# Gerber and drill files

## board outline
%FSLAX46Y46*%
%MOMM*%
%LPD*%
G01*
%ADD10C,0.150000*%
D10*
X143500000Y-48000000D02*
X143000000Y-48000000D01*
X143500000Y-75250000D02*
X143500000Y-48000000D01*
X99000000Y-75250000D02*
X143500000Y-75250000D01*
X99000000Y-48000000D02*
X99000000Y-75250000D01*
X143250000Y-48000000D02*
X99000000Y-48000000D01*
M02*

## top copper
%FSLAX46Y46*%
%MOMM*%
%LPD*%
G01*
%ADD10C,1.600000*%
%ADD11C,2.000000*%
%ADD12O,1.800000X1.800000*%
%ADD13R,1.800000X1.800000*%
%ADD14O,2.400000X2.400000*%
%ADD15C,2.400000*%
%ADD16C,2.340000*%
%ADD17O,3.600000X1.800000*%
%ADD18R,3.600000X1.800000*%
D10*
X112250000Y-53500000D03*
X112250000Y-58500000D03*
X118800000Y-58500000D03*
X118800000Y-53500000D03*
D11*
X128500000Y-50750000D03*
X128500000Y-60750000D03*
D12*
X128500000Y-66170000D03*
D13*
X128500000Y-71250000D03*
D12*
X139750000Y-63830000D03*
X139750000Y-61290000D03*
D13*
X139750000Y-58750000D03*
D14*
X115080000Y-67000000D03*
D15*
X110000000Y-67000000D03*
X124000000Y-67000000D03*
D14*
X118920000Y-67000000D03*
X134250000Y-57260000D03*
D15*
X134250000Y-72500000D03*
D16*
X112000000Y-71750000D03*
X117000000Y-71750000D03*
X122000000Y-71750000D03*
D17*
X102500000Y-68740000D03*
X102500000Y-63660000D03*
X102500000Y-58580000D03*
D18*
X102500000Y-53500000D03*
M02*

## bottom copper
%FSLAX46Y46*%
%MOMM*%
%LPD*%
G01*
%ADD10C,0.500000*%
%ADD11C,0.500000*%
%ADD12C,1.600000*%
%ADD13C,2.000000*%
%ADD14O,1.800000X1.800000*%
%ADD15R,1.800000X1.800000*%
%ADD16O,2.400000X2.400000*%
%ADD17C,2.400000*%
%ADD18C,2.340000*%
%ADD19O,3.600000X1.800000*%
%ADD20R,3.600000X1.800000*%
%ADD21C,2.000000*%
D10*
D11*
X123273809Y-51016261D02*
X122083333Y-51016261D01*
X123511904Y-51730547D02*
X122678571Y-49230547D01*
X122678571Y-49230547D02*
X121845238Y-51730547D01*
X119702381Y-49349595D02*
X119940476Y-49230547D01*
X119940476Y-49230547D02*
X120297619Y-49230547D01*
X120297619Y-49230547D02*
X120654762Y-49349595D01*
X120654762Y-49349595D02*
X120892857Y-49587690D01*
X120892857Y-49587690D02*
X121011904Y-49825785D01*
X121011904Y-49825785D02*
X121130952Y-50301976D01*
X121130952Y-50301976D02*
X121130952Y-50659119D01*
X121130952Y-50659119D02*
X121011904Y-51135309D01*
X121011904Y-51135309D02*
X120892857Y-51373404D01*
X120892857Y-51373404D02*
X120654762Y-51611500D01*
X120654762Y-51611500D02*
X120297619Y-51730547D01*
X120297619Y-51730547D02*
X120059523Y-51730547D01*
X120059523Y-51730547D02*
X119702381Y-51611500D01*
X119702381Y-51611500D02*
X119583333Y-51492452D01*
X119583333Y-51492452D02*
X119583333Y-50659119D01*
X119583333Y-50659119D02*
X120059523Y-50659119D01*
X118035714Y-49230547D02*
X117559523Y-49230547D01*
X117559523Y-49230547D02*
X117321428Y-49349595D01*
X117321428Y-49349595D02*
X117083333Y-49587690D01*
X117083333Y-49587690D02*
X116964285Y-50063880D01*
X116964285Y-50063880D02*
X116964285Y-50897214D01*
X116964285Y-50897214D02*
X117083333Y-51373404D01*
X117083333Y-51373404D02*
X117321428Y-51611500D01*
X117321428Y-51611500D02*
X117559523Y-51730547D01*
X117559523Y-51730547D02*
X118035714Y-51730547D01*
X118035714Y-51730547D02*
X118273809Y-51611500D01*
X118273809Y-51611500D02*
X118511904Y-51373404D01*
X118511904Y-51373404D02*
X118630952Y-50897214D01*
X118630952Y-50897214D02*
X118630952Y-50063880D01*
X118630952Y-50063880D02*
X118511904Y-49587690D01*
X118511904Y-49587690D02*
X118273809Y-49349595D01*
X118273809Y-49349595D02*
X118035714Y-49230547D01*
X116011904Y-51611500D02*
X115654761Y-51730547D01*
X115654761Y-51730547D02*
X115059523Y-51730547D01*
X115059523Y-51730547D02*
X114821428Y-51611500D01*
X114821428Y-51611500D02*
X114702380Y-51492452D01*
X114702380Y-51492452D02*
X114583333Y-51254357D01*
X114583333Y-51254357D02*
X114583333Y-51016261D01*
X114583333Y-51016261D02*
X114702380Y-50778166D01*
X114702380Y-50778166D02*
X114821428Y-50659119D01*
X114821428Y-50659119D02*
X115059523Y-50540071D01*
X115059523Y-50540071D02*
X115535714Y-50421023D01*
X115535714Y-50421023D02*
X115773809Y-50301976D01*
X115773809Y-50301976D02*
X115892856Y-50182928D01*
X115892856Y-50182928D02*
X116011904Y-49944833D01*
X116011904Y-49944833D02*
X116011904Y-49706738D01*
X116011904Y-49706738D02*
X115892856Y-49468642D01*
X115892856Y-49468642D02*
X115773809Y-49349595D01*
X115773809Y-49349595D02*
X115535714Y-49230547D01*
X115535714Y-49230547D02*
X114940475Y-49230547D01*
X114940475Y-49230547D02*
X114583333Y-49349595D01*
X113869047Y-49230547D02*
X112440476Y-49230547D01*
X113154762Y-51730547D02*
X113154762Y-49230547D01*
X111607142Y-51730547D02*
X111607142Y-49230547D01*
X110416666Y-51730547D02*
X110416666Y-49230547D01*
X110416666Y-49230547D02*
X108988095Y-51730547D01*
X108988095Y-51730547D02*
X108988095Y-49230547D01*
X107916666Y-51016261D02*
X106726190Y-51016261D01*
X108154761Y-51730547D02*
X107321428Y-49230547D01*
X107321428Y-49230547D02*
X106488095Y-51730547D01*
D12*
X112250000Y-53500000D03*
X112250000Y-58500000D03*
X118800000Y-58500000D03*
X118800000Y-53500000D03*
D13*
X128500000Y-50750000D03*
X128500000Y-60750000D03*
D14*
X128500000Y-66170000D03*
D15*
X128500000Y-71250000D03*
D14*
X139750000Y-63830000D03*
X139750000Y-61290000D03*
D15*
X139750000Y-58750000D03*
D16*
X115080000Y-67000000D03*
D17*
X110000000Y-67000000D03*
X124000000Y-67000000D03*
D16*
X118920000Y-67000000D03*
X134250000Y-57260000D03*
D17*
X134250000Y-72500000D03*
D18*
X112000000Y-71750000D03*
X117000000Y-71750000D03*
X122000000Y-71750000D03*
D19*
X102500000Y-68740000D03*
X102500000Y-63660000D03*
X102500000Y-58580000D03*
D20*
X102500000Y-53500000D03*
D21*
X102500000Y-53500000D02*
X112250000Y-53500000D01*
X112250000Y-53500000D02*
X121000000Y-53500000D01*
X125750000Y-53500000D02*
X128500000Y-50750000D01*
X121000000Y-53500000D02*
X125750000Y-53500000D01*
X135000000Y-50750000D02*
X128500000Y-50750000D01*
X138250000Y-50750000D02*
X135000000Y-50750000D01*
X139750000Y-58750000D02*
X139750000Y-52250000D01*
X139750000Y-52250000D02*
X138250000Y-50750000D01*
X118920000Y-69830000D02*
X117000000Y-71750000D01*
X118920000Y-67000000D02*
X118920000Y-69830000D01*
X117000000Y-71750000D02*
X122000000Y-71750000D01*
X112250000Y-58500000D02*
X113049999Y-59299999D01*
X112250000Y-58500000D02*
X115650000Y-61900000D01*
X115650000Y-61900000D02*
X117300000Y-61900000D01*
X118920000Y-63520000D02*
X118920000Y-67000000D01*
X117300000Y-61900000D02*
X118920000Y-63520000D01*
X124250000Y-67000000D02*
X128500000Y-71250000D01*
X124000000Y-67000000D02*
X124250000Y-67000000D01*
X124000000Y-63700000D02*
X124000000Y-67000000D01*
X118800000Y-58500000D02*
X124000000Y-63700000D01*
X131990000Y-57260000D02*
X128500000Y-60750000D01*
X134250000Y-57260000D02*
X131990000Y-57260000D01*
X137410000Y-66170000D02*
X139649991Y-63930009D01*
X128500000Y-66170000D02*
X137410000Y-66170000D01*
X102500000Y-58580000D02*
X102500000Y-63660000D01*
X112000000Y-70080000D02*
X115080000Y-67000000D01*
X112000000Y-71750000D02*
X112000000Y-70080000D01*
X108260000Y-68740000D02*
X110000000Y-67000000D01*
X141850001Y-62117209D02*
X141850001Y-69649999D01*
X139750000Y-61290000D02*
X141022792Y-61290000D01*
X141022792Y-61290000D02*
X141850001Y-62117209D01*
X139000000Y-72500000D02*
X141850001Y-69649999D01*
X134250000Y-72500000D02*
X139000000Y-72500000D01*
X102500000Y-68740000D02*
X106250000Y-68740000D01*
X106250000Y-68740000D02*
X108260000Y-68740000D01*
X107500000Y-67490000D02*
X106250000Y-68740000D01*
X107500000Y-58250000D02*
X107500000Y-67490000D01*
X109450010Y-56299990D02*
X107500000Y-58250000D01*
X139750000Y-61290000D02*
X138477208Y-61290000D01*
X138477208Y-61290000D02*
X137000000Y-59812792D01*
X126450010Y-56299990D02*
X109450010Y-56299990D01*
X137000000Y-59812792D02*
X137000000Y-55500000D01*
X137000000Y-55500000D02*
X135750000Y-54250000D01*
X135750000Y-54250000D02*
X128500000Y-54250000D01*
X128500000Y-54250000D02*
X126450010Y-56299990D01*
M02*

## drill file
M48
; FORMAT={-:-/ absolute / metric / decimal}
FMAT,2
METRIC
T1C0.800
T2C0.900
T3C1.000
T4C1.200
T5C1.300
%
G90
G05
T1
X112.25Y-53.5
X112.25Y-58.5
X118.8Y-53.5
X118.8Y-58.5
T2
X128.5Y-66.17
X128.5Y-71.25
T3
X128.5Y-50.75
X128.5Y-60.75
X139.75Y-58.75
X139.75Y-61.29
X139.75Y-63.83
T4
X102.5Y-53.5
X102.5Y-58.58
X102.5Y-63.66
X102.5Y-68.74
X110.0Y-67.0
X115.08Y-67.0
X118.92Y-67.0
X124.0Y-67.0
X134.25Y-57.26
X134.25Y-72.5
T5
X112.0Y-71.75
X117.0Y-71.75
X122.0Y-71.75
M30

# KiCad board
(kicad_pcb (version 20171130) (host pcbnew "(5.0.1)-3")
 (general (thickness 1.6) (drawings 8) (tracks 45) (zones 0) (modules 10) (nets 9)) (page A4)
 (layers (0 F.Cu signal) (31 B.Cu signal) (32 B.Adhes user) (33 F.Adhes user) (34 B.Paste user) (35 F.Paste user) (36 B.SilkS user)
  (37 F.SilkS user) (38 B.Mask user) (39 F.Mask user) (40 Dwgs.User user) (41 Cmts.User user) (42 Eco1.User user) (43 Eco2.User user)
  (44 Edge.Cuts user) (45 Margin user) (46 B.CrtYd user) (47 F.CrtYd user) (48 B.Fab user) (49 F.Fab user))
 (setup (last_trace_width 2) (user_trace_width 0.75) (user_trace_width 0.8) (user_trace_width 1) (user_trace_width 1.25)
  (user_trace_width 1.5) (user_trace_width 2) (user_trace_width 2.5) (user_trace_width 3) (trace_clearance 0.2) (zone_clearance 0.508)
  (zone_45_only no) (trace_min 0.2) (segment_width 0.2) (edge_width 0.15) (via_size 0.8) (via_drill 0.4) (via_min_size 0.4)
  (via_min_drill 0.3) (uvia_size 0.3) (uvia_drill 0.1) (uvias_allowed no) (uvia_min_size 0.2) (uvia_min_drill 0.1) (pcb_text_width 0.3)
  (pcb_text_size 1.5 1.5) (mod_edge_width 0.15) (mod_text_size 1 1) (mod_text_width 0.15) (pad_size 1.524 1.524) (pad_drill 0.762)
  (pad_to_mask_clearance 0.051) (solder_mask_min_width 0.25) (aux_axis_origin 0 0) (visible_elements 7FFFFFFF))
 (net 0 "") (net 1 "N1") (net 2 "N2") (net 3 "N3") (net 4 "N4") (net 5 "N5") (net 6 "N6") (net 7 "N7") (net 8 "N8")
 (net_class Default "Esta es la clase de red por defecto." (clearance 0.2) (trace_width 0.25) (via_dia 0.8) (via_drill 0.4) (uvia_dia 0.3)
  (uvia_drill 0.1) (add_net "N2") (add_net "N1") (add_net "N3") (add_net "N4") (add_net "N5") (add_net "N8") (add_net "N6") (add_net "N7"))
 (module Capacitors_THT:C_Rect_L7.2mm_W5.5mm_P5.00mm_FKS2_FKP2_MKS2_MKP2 (layer F.Cu) (at 112.25 58.5 90)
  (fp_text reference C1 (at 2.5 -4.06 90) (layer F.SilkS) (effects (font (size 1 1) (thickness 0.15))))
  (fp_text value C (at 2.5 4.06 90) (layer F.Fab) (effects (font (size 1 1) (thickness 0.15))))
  (pad 2 thru_hole circle (at 5 0 90) (size 1.6 1.6) (drill 0.8) (layers *.Cu *.Mask) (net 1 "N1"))
  (pad 1 thru_hole circle (at 0 0 90) (size 1.6 1.6) (drill 0.8) (layers *.Cu *.Mask) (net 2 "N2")))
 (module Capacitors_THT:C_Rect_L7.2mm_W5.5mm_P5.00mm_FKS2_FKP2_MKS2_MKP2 (layer F.Cu) (at 118.8 58.5 90)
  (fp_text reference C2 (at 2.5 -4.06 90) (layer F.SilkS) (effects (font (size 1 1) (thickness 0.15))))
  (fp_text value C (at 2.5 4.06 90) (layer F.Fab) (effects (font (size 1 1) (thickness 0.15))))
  (pad 1 thru_hole circle (at 0 0 90) (size 1.6 1.6) (drill 0.8) (layers *.Cu *.Mask) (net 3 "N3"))
  (pad 2 thru_hole circle (at 5 0 90) (size 1.6 1.6) (drill 0.8) (layers *.Cu *.Mask) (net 1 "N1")))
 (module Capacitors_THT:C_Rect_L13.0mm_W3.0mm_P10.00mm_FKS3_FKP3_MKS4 (layer F.Cu) (at 128.5 60.75 90)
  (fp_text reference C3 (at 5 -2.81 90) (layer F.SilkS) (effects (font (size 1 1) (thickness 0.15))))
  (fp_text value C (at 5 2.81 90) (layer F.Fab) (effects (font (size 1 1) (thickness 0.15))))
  (pad 2 thru_hole circle (at 10 0 90) (size 2 2) (drill 1) (layers *.Cu *.Mask) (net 1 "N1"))
  (pad 1 thru_hole circle (at 0 0 90) (size 2 2) (drill 1) (layers *.Cu *.Mask) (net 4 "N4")))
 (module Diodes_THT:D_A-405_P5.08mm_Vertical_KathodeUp (layer F.Cu) (at 128.5 71.25 90)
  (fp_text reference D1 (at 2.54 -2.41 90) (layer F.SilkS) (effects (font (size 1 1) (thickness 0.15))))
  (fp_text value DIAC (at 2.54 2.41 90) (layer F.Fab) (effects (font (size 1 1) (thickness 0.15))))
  (pad 2 thru_hole oval (at 5.08 0 90) (size 1.8 1.8) (drill 0.9) (layers *.Cu *.Mask) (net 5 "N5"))
  (pad 1 thru_hole rect (at 0 0 90) (size 1.8 1.8) (drill 0.9) (layers *.Cu *.Mask) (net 3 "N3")))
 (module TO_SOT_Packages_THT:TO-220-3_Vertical (layer F.Cu) (at 139.75 58.75 270)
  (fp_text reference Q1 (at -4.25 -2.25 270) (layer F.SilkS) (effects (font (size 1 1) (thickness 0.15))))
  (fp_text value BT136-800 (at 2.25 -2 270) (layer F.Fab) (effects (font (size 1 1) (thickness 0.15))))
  (pad 3 thru_hole oval (at 5.08 0 270) (size 1.8 1.8) (drill 1) (layers *.Cu *.Mask) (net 5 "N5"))
  (pad 2 thru_hole oval (at 2.54 0 270) (size 1.8 1.8) (drill 1) (layers *.Cu *.Mask) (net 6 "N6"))
  (pad 1 thru_hole rect (at 0 0 270) (size 1.8 1.8) (drill 1) (layers *.Cu *.Mask) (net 1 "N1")))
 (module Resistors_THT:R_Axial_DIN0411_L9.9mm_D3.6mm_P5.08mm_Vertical (layer F.Cu) (at 110 67)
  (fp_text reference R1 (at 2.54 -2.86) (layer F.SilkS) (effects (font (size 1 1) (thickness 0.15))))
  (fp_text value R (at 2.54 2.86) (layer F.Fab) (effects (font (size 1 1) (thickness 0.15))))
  (pad 2 thru_hole oval (at 5.08 0) (size 2.4 2.4) (drill 1.2) (layers *.Cu *.Mask) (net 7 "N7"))
  (pad 1 thru_hole circle (at 0 0) (size 2.4 2.4) (drill 1.2) (layers *.Cu *.Mask) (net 6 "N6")))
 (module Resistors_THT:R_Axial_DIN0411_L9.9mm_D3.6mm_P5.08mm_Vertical (layer F.Cu) (at 124 67 180)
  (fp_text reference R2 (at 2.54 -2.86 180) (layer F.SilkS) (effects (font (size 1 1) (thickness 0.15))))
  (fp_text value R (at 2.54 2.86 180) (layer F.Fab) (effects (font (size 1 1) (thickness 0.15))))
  (pad 1 thru_hole circle (at 0 0 180) (size 2.4 2.4) (drill 1.2) (layers *.Cu *.Mask) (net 3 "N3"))
  (pad 2 thru_hole oval (at 5.08 0 180) (size 2.4 2.4) (drill 1.2) (layers *.Cu *.Mask) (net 2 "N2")))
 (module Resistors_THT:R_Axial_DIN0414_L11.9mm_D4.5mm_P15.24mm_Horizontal (layer F.Cu) (at 134.25 72.5 90)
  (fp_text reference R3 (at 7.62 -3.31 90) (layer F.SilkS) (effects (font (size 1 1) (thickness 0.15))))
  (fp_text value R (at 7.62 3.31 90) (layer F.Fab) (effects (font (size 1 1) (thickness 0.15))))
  (pad 2 thru_hole oval (at 15.24 0 90) (size 2.4 2.4) (drill 1.2) (layers *.Cu *.Mask) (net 4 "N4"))
  (pad 1 thru_hole circle (at 0 0 90) (size 2.4 2.4) (drill 1.2) (layers *.Cu *.Mask) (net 6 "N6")))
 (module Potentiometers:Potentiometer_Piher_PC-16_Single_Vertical (layer F.Cu) (at 112 71.75 270)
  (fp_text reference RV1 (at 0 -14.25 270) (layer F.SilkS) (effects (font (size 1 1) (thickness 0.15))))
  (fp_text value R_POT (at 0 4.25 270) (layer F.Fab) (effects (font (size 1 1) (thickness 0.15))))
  (pad 1 thru_hole circle (at 0 0 270) (size 2.34 2.34) (drill 1.3) (layers *.Cu *.Mask) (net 7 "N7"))
  (pad 2 thru_hole circle (at 0 -5 270) (size 2.34 2.34) (drill 1.3) (layers *.Cu *.Mask) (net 2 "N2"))
  (pad 3 thru_hole circle (at 0 -10 270) (size 2.34 2.34) (drill 1.3) (layers *.Cu *.Mask) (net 2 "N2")))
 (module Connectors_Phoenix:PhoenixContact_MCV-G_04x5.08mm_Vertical (layer F.Cu) (at 102.5 53.5 270)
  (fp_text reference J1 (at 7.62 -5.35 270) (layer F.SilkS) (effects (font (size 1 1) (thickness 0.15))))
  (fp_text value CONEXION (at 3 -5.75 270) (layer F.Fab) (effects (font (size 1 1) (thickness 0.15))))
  (pad 4 thru_hole oval (at 15.24 0 270) (size 1.8 3.6) (drill 1.2) (layers *.Cu *.Mask) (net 6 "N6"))
  (pad 3 thru_hole oval (at 10.16 0 270) (size 1.8 3.6) (drill 1.2) (layers *.Cu *.Mask) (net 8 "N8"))
  (pad 2 thru_hole oval (at 5.08 0 270) (size 1.8 3.6) (drill 1.2) (layers *.Cu *.Mask) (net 8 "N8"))
  (pad 1 thru_hole rect (at 0 0 270) (size 1.8 3.6) (drill 1.2) (layers *.Cu *.Mask) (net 1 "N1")))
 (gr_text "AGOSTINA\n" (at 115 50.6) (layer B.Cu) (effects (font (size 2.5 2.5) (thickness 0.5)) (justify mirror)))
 (gr_line (start 143.5 48) (end 143 48) (layer Edge.Cuts) (width 0.15))
 (gr_line (start 143.5 75.25) (end 143.5 48) (layer Edge.Cuts) (width 0.15))
 (gr_line (start 99 75.25) (end 143.5 75.25) (layer Edge.Cuts) (width 0.15))
 (gr_line (start 99 48) (end 99 75.25) (layer Edge.Cuts) (width 0.15))
 (gr_line (start 143.25 48) (end 99 48) (layer Edge.Cuts) (width 0.15))
 (segment (start 102.5 53.5) (end 112.25 53.5) (width 2) (layer B.Cu) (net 1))
 (segment (start 112.25 53.5) (end 121 53.5) (width 2) (layer B.Cu) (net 1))
 (segment (start 125.75 53.5) (end 128.5 50.75) (width 2) (layer B.Cu) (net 1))
 (segment (start 121 53.5) (end 125.75 53.5) (width 2) (layer B.Cu) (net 1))
 (segment (start 135 50.75) (end 128.5 50.75) (width 2) (layer B.Cu) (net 1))
 (segment (start 138.25 50.75) (end 135 50.75) (width 2) (layer B.Cu) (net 1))
 (segment (start 139.75 58.75) (end 139.75 52.25) (width 2) (layer B.Cu) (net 1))
 (segment (start 139.75 52.25) (end 138.25 50.75) (width 2) (layer B.Cu) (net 1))
 (segment (start 118.92 69.83) (end 117 71.75) (width 2) (layer B.Cu) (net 2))
 (segment (start 118.92 67) (end 118.92 69.83) (width 2) (layer B.Cu) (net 2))
 (segment (start 117 71.75) (end 122 71.75) (width 2) (layer B.Cu) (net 2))
 (segment (start 112.25 58.5) (end 113.049999 59.299999) (width 2) (layer B.Cu) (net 2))
 (segment (start 112.25 58.5) (end 115.65 61.9) (width 2) (layer B.Cu) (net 2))
 (segment (start 115.65 61.9) (end 117.3 61.9) (width 2) (layer B.Cu) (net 2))
 (segment (start 118.92 63.52) (end 118.92 67) (width 2) (layer B.Cu) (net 2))
 (segment (start 117.3 61.9) (end 118.92 63.52) (width 2) (layer B.Cu) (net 2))
 (segment (start 124.25 67) (end 128.5 71.25) (width 2) (layer B.Cu) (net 3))
 (segment (start 124 67) (end 124.25 67) (width 2) (layer B.Cu) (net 3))
 (segment (start 124 63.7) (end 124 67) (width 2) (layer B.Cu) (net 3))
 (segment (start 118.8 58.5) (end 124 63.7) (width 2) (layer B.Cu) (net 3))
 (segment (start 131.99 57.26) (end 128.5 60.75) (width 2) (layer B.Cu) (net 4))
 (segment (start 134.25 57.26) (end 131.99 57.26) (width 2) (layer B.Cu) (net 4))
 (segment (start 137.41 66.17) (end 139.649991 63.930009) (width 2) (layer B.Cu) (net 5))
 (segment (start 128.5 66.17) (end 137.41 66.17) (width 2) (layer B.Cu) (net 5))
 (segment (start 102.5 58.58) (end 102.5 63.66) (width 2) (layer B.Cu) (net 8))
 (segment (start 112 70.08) (end 115.08 67) (width 2) (layer B.Cu) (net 7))
 (segment (start 112 71.75) (end 112 70.08) (width 2) (layer B.Cu) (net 7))
 (segment (start 108.26 68.74) (end 110 67) (width 2) (layer B.Cu) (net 6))
 (segment (start 141.850001 62.117209) (end 141.850001 69.649999) (width 2) (layer B.Cu) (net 6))
 (segment (start 139.75 61.29) (end 141.022792 61.29) (width 2) (layer B.Cu) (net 6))
 (segment (start 141.022792 61.29) (end 141.850001 62.117209) (width 2) (layer B.Cu) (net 6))
 (segment (start 139 72.5) (end 141.850001 69.649999) (width 2) (layer B.Cu) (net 6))
 (segment (start 134.25 72.5) (end 139 72.5) (width 2) (layer B.Cu) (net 6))
 (segment (start 102.5 68.74) (end 106.25 68.74) (width 2) (layer B.Cu) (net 6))
 (segment (start 106.25 68.74) (end 108.26 68.74) (width 2) (layer B.Cu) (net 6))
 (segment (start 107.5 67.49) (end 106.25 68.74) (width 2) (layer B.Cu) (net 6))
 (segment (start 107.5 58.25) (end 107.5 67.49) (width 2) (layer B.Cu) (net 6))
 (segment (start 109.45001 56.29999) (end 107.5 58.25) (width 2) (layer B.Cu) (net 6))
 (segment (start 139.75 61.29) (end 138.477208 61.29) (width 2) (layer B.Cu) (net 6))
 (segment (start 138.477208 61.29) (end 137 59.812792) (width 2) (layer B.Cu) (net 6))
 (segment (start 126.45001 56.29999) (end 109.45001 56.29999) (width 2) (layer B.Cu) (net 6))
 (segment (start 137 59.812792) (end 137 55.5) (width 2) (layer B.Cu) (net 6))
 (segment (start 137 55.5) (end 135.75 54.25) (width 2) (layer B.Cu) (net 6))
 (segment (start 135.75 54.25) (end 128.5 54.25) (width 2) (layer B.Cu) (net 6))
 (segment (start 128.5 54.25) (end 126.45001 56.29999) (width 2) (layer B.Cu) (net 6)))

